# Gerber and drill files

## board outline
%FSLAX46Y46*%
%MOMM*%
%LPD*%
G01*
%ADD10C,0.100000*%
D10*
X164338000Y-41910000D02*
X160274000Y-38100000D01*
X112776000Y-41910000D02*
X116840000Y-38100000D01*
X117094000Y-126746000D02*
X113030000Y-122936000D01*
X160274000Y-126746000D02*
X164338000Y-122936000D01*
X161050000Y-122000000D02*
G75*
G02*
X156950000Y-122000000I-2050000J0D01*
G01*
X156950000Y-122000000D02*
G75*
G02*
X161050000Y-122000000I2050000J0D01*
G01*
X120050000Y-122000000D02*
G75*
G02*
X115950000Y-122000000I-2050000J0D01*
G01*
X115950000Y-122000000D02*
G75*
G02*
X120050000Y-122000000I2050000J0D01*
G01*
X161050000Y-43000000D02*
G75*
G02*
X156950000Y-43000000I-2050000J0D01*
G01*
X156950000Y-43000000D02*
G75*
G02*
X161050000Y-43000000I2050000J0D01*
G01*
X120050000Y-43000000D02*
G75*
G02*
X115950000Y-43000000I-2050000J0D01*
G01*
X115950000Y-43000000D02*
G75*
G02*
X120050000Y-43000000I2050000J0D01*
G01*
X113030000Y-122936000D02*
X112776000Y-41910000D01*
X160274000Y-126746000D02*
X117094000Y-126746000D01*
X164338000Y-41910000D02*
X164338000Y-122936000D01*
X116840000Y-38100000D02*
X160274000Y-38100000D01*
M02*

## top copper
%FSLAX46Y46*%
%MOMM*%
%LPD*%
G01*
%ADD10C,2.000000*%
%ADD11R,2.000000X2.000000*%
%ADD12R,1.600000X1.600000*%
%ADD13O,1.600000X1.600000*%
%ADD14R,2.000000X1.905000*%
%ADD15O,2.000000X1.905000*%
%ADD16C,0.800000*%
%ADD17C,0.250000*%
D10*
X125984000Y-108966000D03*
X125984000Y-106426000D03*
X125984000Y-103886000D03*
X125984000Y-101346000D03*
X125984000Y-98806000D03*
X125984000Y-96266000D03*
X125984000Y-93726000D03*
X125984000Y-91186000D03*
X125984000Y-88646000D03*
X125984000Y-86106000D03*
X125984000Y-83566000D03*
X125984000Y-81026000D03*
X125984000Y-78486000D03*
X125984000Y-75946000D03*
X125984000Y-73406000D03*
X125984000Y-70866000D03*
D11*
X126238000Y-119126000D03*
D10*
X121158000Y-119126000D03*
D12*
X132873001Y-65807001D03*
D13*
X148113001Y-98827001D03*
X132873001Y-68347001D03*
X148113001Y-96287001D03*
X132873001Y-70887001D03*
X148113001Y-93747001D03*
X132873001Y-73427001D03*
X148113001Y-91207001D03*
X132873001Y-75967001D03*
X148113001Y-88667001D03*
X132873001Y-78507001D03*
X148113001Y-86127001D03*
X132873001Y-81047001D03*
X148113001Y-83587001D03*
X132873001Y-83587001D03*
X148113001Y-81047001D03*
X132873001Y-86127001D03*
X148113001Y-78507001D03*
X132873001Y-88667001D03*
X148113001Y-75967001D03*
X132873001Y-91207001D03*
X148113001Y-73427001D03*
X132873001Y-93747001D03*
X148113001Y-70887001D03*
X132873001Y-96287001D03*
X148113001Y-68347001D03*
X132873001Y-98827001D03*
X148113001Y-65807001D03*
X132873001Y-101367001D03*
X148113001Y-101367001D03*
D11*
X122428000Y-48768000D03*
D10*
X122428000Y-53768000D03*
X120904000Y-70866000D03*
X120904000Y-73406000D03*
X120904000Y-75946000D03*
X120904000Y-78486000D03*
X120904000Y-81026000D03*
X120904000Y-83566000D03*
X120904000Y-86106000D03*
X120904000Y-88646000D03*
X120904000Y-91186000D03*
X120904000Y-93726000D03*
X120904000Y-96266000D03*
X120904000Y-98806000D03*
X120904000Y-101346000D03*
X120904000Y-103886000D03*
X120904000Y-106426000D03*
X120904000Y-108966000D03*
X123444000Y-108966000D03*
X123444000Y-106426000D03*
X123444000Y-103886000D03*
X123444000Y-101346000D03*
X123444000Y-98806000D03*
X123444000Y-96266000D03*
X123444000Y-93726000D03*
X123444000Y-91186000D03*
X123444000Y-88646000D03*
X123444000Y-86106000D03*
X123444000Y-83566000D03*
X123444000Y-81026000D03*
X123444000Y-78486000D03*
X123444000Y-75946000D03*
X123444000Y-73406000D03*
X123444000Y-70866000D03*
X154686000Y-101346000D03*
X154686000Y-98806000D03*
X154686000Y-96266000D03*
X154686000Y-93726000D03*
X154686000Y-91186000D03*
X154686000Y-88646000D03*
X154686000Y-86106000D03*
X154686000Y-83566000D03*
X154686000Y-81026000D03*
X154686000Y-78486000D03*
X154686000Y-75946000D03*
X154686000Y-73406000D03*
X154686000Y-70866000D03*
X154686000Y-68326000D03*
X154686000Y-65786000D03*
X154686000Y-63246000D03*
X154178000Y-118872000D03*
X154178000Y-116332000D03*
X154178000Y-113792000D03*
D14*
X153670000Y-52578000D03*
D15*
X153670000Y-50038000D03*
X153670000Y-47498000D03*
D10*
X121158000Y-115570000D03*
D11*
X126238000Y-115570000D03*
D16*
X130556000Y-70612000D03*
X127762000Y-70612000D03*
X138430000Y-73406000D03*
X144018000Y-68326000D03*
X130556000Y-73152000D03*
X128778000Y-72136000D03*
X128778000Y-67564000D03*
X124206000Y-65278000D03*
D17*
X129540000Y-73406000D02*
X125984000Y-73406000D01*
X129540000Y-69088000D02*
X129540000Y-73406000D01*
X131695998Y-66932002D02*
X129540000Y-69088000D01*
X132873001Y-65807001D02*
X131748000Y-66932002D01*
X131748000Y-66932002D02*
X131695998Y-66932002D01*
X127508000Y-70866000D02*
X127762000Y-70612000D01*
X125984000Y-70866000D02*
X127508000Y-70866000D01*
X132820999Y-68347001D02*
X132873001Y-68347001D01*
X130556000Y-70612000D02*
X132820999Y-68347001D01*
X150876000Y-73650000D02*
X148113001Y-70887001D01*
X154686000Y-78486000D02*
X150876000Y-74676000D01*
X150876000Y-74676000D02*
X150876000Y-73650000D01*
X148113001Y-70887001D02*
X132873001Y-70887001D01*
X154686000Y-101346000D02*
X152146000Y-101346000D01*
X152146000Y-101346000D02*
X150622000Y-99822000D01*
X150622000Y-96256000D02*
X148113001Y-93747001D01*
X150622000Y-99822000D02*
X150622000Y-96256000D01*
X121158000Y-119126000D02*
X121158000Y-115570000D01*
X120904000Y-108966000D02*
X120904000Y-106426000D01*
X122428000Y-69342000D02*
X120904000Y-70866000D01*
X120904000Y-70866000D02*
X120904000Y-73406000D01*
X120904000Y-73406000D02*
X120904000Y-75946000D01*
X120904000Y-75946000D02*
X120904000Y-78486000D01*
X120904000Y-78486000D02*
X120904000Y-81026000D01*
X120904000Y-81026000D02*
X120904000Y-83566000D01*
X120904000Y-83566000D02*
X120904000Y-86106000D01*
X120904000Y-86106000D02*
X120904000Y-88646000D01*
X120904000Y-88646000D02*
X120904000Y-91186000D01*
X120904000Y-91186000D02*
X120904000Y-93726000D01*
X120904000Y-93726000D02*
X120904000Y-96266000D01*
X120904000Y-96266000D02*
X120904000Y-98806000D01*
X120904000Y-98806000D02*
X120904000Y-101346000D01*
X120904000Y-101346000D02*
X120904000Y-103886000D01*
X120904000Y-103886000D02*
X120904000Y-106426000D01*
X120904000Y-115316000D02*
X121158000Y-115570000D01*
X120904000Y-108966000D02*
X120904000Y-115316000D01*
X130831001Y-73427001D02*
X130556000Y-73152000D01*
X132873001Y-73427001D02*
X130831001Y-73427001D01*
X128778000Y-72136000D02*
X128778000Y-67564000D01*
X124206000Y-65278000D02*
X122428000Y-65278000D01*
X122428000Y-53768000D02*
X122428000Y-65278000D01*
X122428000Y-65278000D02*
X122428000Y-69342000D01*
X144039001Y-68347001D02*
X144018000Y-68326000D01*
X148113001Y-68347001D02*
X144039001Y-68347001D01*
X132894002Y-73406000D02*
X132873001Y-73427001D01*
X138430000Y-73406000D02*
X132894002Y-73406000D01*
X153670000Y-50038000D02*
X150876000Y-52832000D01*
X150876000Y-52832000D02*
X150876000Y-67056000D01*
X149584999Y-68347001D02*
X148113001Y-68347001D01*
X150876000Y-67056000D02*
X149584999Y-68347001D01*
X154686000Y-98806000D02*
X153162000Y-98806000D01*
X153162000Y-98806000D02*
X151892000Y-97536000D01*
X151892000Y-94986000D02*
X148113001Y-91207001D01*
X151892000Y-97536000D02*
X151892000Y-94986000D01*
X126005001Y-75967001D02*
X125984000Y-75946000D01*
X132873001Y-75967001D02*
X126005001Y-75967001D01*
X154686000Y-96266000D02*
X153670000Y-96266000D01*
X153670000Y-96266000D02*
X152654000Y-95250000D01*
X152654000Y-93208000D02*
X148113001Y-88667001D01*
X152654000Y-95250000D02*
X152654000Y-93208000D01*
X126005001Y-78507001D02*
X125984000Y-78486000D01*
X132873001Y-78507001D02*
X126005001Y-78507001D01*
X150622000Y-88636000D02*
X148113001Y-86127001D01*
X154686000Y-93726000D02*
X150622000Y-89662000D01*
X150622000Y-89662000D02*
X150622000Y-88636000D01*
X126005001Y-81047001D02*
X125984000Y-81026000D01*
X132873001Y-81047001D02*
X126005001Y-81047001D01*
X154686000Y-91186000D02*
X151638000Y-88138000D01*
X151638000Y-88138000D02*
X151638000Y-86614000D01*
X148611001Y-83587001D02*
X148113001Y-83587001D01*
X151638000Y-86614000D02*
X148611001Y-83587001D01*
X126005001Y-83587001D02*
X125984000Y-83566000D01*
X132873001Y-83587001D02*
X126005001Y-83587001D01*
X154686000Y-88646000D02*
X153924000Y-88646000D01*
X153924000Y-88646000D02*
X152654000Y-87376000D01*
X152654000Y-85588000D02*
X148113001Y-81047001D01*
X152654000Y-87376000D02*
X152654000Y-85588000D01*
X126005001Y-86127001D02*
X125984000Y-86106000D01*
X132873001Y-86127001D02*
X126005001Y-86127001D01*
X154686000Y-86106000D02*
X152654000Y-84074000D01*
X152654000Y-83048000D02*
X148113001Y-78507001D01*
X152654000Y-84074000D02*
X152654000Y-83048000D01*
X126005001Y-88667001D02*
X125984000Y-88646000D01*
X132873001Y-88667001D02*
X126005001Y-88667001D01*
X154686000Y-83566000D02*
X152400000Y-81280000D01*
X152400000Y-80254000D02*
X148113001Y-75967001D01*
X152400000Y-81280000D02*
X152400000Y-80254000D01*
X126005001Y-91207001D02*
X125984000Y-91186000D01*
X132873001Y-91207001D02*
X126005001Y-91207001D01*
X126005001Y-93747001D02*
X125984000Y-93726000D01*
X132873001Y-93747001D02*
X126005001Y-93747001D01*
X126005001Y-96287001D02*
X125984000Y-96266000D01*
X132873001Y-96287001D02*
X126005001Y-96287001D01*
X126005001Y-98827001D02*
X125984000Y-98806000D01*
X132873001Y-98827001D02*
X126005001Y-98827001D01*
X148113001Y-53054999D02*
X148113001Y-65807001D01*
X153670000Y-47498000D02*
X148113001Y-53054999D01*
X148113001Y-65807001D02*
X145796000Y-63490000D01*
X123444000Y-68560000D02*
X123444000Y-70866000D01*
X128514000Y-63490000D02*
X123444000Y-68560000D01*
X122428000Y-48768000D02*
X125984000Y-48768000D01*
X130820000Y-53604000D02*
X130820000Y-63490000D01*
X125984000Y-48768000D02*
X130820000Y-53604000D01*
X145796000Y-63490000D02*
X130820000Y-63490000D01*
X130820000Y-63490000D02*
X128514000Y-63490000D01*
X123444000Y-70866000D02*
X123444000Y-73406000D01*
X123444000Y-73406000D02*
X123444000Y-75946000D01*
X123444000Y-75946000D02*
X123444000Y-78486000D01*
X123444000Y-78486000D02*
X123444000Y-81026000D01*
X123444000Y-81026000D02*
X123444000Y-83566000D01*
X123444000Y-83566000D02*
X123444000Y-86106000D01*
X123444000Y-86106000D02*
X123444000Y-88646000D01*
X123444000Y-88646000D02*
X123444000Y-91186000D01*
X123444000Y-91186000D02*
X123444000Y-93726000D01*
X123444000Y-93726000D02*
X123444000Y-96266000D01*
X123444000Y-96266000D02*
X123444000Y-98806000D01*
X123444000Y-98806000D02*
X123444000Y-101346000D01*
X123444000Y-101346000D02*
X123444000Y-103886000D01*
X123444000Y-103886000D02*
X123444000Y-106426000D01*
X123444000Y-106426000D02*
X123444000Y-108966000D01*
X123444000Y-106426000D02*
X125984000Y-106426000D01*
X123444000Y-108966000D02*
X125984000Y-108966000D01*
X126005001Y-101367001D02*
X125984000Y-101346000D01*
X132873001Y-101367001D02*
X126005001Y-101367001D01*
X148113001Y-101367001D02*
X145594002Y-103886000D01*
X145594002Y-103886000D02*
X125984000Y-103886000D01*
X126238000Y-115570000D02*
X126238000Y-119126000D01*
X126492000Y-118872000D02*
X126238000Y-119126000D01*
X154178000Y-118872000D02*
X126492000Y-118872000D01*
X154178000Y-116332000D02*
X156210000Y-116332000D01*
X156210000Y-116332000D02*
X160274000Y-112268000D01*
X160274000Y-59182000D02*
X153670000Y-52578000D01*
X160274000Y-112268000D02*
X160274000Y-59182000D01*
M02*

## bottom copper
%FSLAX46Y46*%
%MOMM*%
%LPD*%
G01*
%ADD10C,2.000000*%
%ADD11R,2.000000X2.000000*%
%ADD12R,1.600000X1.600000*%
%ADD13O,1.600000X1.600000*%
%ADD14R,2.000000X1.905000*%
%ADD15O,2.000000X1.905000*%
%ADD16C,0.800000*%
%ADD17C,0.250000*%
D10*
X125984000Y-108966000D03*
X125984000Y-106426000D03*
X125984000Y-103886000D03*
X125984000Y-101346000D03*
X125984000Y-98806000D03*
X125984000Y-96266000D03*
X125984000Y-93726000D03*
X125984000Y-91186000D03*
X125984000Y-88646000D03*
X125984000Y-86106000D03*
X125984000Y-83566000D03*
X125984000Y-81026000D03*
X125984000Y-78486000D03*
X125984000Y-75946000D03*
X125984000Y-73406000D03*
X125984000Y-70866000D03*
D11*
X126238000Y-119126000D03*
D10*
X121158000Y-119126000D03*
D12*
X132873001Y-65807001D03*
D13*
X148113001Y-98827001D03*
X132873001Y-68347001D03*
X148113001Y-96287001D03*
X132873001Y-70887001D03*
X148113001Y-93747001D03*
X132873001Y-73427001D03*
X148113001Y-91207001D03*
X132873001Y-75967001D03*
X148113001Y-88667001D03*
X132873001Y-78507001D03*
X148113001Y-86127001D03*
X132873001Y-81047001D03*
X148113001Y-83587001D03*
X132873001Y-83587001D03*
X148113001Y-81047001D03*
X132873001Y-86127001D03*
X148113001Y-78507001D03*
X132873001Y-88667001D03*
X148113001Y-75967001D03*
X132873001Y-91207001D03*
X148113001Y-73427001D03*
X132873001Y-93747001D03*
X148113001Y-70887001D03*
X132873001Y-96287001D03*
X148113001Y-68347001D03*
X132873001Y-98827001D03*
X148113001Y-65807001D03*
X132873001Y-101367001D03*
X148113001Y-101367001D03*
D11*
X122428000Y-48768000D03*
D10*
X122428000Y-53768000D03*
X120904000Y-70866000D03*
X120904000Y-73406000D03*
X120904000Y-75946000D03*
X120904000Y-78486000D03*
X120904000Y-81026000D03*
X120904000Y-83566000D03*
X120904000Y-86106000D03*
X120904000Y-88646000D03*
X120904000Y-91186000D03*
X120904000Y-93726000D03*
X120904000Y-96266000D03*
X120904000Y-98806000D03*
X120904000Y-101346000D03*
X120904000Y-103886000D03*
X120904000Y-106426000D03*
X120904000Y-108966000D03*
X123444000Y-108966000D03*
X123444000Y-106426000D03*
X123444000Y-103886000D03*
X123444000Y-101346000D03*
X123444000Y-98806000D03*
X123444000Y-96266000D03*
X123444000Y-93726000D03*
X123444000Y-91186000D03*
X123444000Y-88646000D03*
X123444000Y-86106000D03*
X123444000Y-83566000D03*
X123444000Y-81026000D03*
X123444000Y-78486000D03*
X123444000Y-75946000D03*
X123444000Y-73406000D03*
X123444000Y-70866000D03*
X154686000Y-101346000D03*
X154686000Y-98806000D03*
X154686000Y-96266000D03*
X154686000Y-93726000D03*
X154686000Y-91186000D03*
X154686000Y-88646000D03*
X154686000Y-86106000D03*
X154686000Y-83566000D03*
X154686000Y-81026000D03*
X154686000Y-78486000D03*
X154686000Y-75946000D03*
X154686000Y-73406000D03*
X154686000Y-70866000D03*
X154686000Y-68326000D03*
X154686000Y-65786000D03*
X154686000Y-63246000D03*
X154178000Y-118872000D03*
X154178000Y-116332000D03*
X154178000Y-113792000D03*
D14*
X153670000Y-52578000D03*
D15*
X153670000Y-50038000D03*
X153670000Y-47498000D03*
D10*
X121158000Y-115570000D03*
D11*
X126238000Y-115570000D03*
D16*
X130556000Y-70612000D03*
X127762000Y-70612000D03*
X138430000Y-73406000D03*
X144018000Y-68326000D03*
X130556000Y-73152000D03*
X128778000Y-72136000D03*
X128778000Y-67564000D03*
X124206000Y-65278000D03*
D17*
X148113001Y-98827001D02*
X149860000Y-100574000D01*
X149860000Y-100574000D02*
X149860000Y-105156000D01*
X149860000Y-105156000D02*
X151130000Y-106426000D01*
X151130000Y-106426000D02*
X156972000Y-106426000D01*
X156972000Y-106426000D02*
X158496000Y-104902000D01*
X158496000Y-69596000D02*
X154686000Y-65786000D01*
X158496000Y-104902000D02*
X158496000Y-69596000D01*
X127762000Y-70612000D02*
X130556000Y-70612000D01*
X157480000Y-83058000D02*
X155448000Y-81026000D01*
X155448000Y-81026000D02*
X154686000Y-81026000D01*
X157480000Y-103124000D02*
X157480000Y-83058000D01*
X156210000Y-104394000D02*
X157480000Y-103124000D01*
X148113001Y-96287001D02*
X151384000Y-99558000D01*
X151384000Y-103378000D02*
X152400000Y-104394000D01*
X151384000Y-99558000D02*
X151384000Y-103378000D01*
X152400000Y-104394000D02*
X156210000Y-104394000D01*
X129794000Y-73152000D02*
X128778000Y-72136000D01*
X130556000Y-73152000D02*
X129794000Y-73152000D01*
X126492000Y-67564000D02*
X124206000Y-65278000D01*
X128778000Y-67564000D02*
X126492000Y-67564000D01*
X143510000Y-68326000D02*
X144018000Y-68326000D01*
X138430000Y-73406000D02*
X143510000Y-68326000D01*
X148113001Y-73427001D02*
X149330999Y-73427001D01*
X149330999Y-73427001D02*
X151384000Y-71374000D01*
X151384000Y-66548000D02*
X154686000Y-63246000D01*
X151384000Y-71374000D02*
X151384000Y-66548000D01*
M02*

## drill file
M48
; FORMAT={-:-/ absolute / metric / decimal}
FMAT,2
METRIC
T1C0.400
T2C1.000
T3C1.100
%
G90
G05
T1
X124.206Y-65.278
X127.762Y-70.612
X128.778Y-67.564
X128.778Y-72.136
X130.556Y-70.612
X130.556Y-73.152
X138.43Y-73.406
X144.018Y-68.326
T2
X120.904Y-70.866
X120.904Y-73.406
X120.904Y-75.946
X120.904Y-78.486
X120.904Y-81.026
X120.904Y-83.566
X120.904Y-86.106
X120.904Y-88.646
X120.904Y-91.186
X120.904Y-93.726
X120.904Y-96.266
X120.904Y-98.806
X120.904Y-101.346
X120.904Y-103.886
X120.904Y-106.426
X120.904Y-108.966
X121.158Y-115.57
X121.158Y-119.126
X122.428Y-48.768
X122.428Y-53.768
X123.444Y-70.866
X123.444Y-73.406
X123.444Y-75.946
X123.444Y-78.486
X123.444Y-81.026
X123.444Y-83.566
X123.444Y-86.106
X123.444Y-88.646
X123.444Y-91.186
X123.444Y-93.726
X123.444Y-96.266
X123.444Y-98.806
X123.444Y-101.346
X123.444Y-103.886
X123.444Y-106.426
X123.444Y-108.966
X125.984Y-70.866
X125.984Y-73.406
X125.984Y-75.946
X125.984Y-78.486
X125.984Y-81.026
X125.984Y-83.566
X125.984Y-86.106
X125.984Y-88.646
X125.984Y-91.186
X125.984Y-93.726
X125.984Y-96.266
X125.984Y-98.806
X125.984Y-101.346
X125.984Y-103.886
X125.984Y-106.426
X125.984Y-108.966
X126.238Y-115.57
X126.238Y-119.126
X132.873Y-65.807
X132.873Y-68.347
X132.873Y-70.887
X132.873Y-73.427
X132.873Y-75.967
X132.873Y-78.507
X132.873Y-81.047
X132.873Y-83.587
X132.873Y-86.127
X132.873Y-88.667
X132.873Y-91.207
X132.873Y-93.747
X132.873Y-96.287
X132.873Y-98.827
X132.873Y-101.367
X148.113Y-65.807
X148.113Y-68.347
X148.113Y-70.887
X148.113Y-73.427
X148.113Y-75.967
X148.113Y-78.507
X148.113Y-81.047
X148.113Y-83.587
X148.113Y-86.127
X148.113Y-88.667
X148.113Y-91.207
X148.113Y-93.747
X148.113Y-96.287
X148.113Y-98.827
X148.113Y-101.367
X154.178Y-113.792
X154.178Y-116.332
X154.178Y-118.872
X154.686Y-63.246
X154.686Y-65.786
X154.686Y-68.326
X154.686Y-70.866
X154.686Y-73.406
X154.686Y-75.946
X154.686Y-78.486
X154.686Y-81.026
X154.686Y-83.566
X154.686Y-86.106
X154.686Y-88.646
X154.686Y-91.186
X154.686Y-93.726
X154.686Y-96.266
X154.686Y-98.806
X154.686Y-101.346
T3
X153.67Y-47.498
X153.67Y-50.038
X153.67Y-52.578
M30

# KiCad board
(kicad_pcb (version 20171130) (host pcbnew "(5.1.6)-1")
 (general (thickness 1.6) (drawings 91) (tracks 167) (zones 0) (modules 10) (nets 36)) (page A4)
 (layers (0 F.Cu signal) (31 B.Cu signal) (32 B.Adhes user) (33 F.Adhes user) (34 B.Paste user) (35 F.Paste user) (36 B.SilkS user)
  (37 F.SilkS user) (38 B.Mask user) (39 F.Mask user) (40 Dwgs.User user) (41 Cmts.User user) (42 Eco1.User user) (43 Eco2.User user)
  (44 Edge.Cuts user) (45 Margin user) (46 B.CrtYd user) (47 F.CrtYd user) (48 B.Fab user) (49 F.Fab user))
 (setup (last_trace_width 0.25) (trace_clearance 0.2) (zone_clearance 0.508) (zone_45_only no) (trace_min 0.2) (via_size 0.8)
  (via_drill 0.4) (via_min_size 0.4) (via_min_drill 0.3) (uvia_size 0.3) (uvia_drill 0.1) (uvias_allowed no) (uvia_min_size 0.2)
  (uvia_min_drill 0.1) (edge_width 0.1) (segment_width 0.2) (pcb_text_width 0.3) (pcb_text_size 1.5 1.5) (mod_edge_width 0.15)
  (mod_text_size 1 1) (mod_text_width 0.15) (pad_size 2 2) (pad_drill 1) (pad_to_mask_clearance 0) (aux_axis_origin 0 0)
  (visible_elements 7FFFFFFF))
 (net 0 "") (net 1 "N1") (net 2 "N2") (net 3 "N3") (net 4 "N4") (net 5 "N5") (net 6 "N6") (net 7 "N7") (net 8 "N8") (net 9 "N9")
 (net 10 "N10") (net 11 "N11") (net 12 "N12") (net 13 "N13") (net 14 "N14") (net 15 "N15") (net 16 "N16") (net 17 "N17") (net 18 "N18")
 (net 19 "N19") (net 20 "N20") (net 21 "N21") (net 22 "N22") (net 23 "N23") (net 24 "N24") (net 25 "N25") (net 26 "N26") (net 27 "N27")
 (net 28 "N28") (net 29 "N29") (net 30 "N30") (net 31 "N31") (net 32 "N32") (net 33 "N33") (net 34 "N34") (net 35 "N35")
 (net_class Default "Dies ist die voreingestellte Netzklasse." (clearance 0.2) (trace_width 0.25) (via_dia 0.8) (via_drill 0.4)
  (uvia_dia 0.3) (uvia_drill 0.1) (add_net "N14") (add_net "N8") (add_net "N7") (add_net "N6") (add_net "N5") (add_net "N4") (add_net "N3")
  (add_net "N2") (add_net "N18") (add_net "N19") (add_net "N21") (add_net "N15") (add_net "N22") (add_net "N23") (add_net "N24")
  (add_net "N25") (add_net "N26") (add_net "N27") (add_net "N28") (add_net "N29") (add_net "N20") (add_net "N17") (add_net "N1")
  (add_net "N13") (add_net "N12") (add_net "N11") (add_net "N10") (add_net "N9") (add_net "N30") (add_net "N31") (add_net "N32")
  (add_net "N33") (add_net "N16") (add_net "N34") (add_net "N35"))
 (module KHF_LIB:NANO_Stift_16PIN (layer F.Cu) (at 125.984 70.866 270)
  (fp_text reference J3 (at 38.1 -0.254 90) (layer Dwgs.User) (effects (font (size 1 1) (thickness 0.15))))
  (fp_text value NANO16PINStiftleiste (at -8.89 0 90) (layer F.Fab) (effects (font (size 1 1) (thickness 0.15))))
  (pad 16 thru_hole circle (at 38.1 0 270) (size 2 2) (drill 1) (layers *.Cu *.Mask) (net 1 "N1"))
  (pad 15 thru_hole circle (at 35.56 0 270) (size 2 2) (drill 1) (layers *.Cu *.Mask) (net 1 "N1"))
  (pad 14 thru_hole circle (at 33.02 0 270) (size 2 2) (drill 1) (layers *.Cu *.Mask) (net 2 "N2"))
  (pad 13 thru_hole circle (at 30.48 0 270) (size 2 2) (drill 1) (layers *.Cu *.Mask) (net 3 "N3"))
  (pad 12 thru_hole circle (at 27.94 0 270) (size 2 2) (drill 1) (layers *.Cu *.Mask) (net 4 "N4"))
  (pad 11 thru_hole circle (at 25.4 0 270) (size 2 2) (drill 1) (layers *.Cu *.Mask) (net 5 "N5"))
  (pad 10 thru_hole circle (at 22.86 0 270) (size 2 2) (drill 1) (layers *.Cu *.Mask) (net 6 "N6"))
  (pad 9 thru_hole circle (at 20.32 0 270) (size 2 2) (drill 1) (layers *.Cu *.Mask) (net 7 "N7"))
  (pad 8 thru_hole circle (at 17.78 0 270) (size 2 2) (drill 1) (layers *.Cu *.Mask) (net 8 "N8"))
  (pad 7 thru_hole circle (at 15.24 0 270) (size 2 2) (drill 1) (layers *.Cu *.Mask) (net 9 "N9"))
  (pad 6 thru_hole circle (at 12.7 0 270) (size 2 2) (drill 1) (layers *.Cu *.Mask) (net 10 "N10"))
  (pad 5 thru_hole circle (at 10.16 0 270) (size 2 2) (drill 1) (layers *.Cu *.Mask) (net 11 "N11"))
  (pad 4 thru_hole circle (at 7.62 0 270) (size 2 2) (drill 1) (layers *.Cu *.Mask) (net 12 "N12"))
  (pad 3 thru_hole circle (at 5.08 0 270) (size 2 2) (drill 1) (layers *.Cu *.Mask) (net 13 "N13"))
  (pad 2 thru_hole circle (at 2.54 0 270) (size 2 2) (drill 1) (layers *.Cu *.Mask) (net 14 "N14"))
  (pad 1 thru_hole circle (at 0 0 270) (size 2 2) (drill 1) (layers *.Cu *.Mask) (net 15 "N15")))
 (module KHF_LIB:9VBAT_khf (layer F.Cu) (at 121.158 119.126)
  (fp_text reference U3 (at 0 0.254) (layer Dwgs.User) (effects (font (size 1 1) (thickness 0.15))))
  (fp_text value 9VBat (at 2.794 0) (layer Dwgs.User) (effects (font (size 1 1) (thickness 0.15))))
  (pad 2 thru_hole rect (at 5.08 0) (size 2 2) (drill 1) (layers *.Cu *.Mask) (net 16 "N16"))
  (pad 1 thru_hole circle (at 0 0) (size 2 2) (drill 1) (layers *.Cu *.Mask) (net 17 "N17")))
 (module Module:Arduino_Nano (layer F.Cu) (at 132.873001 65.807001)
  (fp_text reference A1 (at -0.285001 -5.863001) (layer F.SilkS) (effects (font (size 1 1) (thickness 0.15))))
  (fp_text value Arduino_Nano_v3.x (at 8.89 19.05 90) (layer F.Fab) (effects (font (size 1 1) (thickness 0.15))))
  (pad 1 thru_hole rect (at 0 0) (size 1.6 1.6) (drill 1) (layers *.Cu *.Mask) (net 14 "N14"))
  (pad 17 thru_hole oval (at 15.24 33.02) (size 1.6 1.6) (drill 1) (layers *.Cu *.Mask) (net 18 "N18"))
  (pad 2 thru_hole oval (at 0 2.54) (size 1.6 1.6) (drill 1) (layers *.Cu *.Mask) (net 15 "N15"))
  (pad 18 thru_hole oval (at 15.24 30.48) (size 1.6 1.6) (drill 1) (layers *.Cu *.Mask) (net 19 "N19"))
  (pad 3 thru_hole oval (at 0 5.08) (size 1.6 1.6) (drill 1) (layers *.Cu *.Mask) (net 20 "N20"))
  (pad 19 thru_hole oval (at 15.24 27.94) (size 1.6 1.6) (drill 1) (layers *.Cu *.Mask) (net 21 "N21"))
  (pad 4 thru_hole oval (at 0 7.62) (size 1.6 1.6) (drill 1) (layers *.Cu *.Mask) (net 17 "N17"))
  (pad 20 thru_hole oval (at 15.24 25.4) (size 1.6 1.6) (drill 1) (layers *.Cu *.Mask) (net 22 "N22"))
  (pad 5 thru_hole oval (at 0 10.16) (size 1.6 1.6) (drill 1) (layers *.Cu *.Mask) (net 13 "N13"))
  (pad 21 thru_hole oval (at 15.24 22.86) (size 1.6 1.6) (drill 1) (layers *.Cu *.Mask) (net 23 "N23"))
  (pad 6 thru_hole oval (at 0 12.7) (size 1.6 1.6) (drill 1) (layers *.Cu *.Mask) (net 12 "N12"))
  (pad 22 thru_hole oval (at 15.24 20.32) (size 1.6 1.6) (drill 1) (layers *.Cu *.Mask) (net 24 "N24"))
  (pad 7 thru_hole oval (at 0 15.24) (size 1.6 1.6) (drill 1) (layers *.Cu *.Mask) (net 11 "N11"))
  (pad 23 thru_hole oval (at 15.24 17.78) (size 1.6 1.6) (drill 1) (layers *.Cu *.Mask) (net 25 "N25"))
  (pad 8 thru_hole oval (at 0 17.78) (size 1.6 1.6) (drill 1) (layers *.Cu *.Mask) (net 10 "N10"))
  (pad 24 thru_hole oval (at 15.24 15.24) (size 1.6 1.6) (drill 1) (layers *.Cu *.Mask) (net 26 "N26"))
  (pad 9 thru_hole oval (at 0 20.32) (size 1.6 1.6) (drill 1) (layers *.Cu *.Mask) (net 9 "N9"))
  (pad 25 thru_hole oval (at 15.24 12.7) (size 1.6 1.6) (drill 1) (layers *.Cu *.Mask) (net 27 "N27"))
  (pad 10 thru_hole oval (at 0 22.86) (size 1.6 1.6) (drill 1) (layers *.Cu *.Mask) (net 8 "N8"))
  (pad 26 thru_hole oval (at 15.24 10.16) (size 1.6 1.6) (drill 1) (layers *.Cu *.Mask) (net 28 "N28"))
  (pad 11 thru_hole oval (at 0 25.4) (size 1.6 1.6) (drill 1) (layers *.Cu *.Mask) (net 7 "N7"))
  (pad 27 thru_hole oval (at 15.24 7.62) (size 1.6 1.6) (drill 1) (layers *.Cu *.Mask) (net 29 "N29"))
  (pad 12 thru_hole oval (at 0 27.94) (size 1.6 1.6) (drill 1) (layers *.Cu *.Mask) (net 6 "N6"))
  (pad 28 thru_hole oval (at 15.24 5.08) (size 1.6 1.6) (drill 1) (layers *.Cu *.Mask) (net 20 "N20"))
  (pad 13 thru_hole oval (at 0 30.48) (size 1.6 1.6) (drill 1) (layers *.Cu *.Mask) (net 5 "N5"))
  (pad 29 thru_hole oval (at 15.24 2.54) (size 1.6 1.6) (drill 1) (layers *.Cu *.Mask) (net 17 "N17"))
  (pad 14 thru_hole oval (at 0 33.02) (size 1.6 1.6) (drill 1) (layers *.Cu *.Mask) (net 4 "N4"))
  (pad 30 thru_hole oval (at 15.24 0) (size 1.6 1.6) (drill 1) (layers *.Cu *.Mask) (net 1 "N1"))
  (pad 15 thru_hole oval (at 0 35.56) (size 1.6 1.6) (drill 1) (layers *.Cu *.Mask) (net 3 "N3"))
  (pad 16 thru_hole oval (at 15.24 35.56) (size 1.6 1.6) (drill 1) (layers *.Cu *.Mask) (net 2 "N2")))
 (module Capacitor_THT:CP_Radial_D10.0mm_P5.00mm (layer F.Cu) (at 122.428 48.768 270)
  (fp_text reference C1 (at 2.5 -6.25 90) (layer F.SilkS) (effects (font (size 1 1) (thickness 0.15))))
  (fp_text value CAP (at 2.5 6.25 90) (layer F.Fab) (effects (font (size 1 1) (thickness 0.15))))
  (pad 1 thru_hole rect (at 0 0 270) (size 2 2) (drill 1) (layers *.Cu *.Mask) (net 1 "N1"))
  (pad 2 thru_hole circle (at 5 0 270) (size 2 2) (drill 1) (layers *.Cu *.Mask) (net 17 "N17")))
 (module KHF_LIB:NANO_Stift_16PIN (layer F.Cu) (at 120.904 70.866 270)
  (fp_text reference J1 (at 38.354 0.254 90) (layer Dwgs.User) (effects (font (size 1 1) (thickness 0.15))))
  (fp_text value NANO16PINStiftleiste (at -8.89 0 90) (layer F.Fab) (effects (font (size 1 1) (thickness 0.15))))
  (pad 1 thru_hole circle (at 0 0 270) (size 2 2) (drill 1) (layers *.Cu *.Mask) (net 17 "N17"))
  (pad 2 thru_hole circle (at 2.54 0 270) (size 2 2) (drill 1) (layers *.Cu *.Mask) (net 17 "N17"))
  (pad 3 thru_hole circle (at 5.08 0 270) (size 2 2) (drill 1) (layers *.Cu *.Mask) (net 17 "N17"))
  (pad 4 thru_hole circle (at 7.62 0 270) (size 2 2) (drill 1) (layers *.Cu *.Mask) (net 17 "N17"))
  (pad 5 thru_hole circle (at 10.16 0 270) (size 2 2) (drill 1) (layers *.Cu *.Mask) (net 17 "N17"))
  (pad 6 thru_hole circle (at 12.7 0 270) (size 2 2) (drill 1) (layers *.Cu *.Mask) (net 17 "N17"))
  (pad 7 thru_hole circle (at 15.24 0 270) (size 2 2) (drill 1) (layers *.Cu *.Mask) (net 17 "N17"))
  (pad 8 thru_hole circle (at 17.78 0 270) (size 2 2) (drill 1) (layers *.Cu *.Mask) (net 17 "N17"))
  (pad 9 thru_hole circle (at 20.32 0 270) (size 2 2) (drill 1) (layers *.Cu *.Mask) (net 17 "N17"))
  (pad 10 thru_hole circle (at 22.86 0 270) (size 2 2) (drill 1) (layers *.Cu *.Mask) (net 17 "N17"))
  (pad 11 thru_hole circle (at 25.4 0 270) (size 2 2) (drill 1) (layers *.Cu *.Mask) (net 17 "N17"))
  (pad 12 thru_hole circle (at 27.94 0 270) (size 2 2) (drill 1) (layers *.Cu *.Mask) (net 17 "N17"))
  (pad 13 thru_hole circle (at 30.48 0 270) (size 2 2) (drill 1) (layers *.Cu *.Mask) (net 17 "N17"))
  (pad 14 thru_hole circle (at 33.02 0 270) (size 2 2) (drill 1) (layers *.Cu *.Mask) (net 17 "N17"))
  (pad 15 thru_hole circle (at 35.56 0 270) (size 2 2) (drill 1) (layers *.Cu *.Mask) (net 17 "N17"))
  (pad 16 thru_hole circle (at 38.1 0 270) (size 2 2) (drill 1) (layers *.Cu *.Mask) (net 17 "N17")))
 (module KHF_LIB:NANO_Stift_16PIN (layer F.Cu) (at 123.444 70.866 270)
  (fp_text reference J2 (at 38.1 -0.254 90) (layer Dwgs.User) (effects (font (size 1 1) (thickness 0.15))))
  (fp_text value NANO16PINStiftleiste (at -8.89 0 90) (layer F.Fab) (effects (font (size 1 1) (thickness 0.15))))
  (pad 16 thru_hole circle (at 38.1 0 270) (size 2 2) (drill 1) (layers *.Cu *.Mask) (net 1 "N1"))
  (pad 15 thru_hole circle (at 35.56 0 270) (size 2 2) (drill 1) (layers *.Cu *.Mask) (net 1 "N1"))
  (pad 14 thru_hole circle (at 33.02 0 270) (size 2 2) (drill 1) (layers *.Cu *.Mask) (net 1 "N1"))
  (pad 13 thru_hole circle (at 30.48 0 270) (size 2 2) (drill 1) (layers *.Cu *.Mask) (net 1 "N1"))
  (pad 12 thru_hole circle (at 27.94 0 270) (size 2 2) (drill 1) (layers *.Cu *.Mask) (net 1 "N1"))
  (pad 11 thru_hole circle (at 25.4 0 270) (size 2 2) (drill 1) (layers *.Cu *.Mask) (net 1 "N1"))
  (pad 10 thru_hole circle (at 22.86 0 270) (size 2 2) (drill 1) (layers *.Cu *.Mask) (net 1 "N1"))
  (pad 9 thru_hole circle (at 20.32 0 270) (size 2 2) (drill 1) (layers *.Cu *.Mask) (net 1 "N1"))
  (pad 8 thru_hole circle (at 17.78 0 270) (size 2 2) (drill 1) (layers *.Cu *.Mask) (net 1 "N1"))
  (pad 7 thru_hole circle (at 15.24 0 270) (size 2 2) (drill 1) (layers *.Cu *.Mask) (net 1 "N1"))
  (pad 6 thru_hole circle (at 12.7 0 270) (size 2 2) (drill 1) (layers *.Cu *.Mask) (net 1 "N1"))
  (pad 5 thru_hole circle (at 10.16 0 270) (size 2 2) (drill 1) (layers *.Cu *.Mask) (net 1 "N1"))
  (pad 4 thru_hole circle (at 7.62 0 270) (size 2 2) (drill 1) (layers *.Cu *.Mask) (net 1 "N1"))
  (pad 3 thru_hole circle (at 5.08 0 270) (size 2 2) (drill 1) (layers *.Cu *.Mask) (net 1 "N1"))
  (pad 2 thru_hole circle (at 2.54 0 270) (size 2 2) (drill 1) (layers *.Cu *.Mask) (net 1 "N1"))
  (pad 1 thru_hole circle (at 0 0 270) (size 2 2) (drill 1) (layers *.Cu *.Mask) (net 1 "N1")))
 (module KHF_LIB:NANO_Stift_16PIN (layer F.Cu) (at 154.686 101.346 90)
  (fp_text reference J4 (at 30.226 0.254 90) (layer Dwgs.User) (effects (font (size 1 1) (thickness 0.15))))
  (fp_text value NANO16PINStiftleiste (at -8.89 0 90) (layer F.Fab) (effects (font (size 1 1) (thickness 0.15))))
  (pad 1 thru_hole circle (at 0 0 90) (size 2 2) (drill 1) (layers *.Cu *.Mask) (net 21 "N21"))
  (pad 2 thru_hole circle (at 2.54 0 90) (size 2 2) (drill 1) (layers *.Cu *.Mask) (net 22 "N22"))
  (pad 3 thru_hole circle (at 5.08 0 90) (size 2 2) (drill 1) (layers *.Cu *.Mask) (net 23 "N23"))
  (pad 4 thru_hole circle (at 7.62 0 90) (size 2 2) (drill 1) (layers *.Cu *.Mask) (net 24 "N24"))
  (pad 5 thru_hole circle (at 10.16 0 90) (size 2 2) (drill 1) (layers *.Cu *.Mask) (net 25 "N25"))
  (pad 6 thru_hole circle (at 12.7 0 90) (size 2 2) (drill 1) (layers *.Cu *.Mask) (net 26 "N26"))
  (pad 7 thru_hole circle (at 15.24 0 90) (size 2 2) (drill 1) (layers *.Cu *.Mask) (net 27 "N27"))
  (pad 8 thru_hole circle (at 17.78 0 90) (size 2 2) (drill 1) (layers *.Cu *.Mask) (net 28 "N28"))
  (pad 9 thru_hole circle (at 20.32 0 90) (size 2 2) (drill 1) (layers *.Cu *.Mask) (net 19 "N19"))
  (pad 10 thru_hole circle (at 22.86 0 90) (size 2 2) (drill 1) (layers *.Cu *.Mask) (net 20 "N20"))
  (pad 11 thru_hole circle (at 25.4 0 90) (size 2 2) (drill 1) (layers *.Cu *.Mask) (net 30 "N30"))
  (pad 12 thru_hole circle (at 27.94 0 90) (size 2 2) (drill 1) (layers *.Cu *.Mask) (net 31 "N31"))
  (pad 13 thru_hole circle (at 30.48 0 90) (size 2 2) (drill 1) (layers *.Cu *.Mask) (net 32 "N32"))
  (pad 14 thru_hole circle (at 33.02 0 90) (size 2 2) (drill 1) (layers *.Cu *.Mask) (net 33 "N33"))
  (pad 15 thru_hole circle (at 35.56 0 90) (size 2 2) (drill 1) (layers *.Cu *.Mask) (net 18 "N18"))
  (pad 16 thru_hole circle (at 38.1 0 90) (size 2 2) (drill 1) (layers *.Cu *.Mask) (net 29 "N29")))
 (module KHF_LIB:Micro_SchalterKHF (layer F.Cu) (at 154.178 118.872 90)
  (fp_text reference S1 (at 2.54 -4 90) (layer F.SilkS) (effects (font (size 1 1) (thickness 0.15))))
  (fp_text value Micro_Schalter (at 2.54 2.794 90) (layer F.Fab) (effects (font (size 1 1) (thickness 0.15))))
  (pad 1 thru_hole circle (at 0 0 90) (size 2 2) (drill 1) (layers *.Cu *.Mask) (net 16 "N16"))
  (pad 2 thru_hole circle (at 2.54 0 90) (size 2 2) (drill 1) (layers *.Cu *.Mask) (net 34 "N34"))
  (pad 3 thru_hole circle (at 5.08 0 90) (size 2 2) (drill 1) (layers *.Cu *.Mask) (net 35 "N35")))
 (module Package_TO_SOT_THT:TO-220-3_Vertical (layer F.Cu) (at 153.67 52.578 90)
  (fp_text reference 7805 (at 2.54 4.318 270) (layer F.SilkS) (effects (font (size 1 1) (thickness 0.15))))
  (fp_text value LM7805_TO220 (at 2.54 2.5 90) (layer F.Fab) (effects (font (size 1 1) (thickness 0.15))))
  (pad 1 thru_hole rect (at 0 0 90) (size 1.905 2) (drill 1.1) (layers *.Cu *.Mask) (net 34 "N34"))
  (pad 2 thru_hole oval (at 2.54 0 90) (size 1.905 2) (drill 1.1) (layers *.Cu *.Mask) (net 17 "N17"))
  (pad 3 thru_hole oval (at 5.08 0 90) (size 1.905 2) (drill 1.1) (layers *.Cu *.Mask) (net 1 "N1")))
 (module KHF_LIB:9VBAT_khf (layer F.Cu) (at 121.158 115.57)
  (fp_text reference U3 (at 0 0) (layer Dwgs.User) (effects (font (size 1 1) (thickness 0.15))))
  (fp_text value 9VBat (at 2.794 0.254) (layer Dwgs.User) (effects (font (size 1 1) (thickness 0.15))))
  (pad 1 thru_hole circle (at 0 0) (size 2 2) (drill 1) (layers *.Cu *.Mask) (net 17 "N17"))
  (pad 2 thru_hole rect (at 5.08 0) (size 2 2) (drill 1) (layers *.Cu *.Mask) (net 16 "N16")))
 (gr_line (start 164.338 41.91) (end 160.274 38.1) (layer Edge.Cuts) (width 0.1))
 (gr_line (start 112.776 41.91) (end 116.84 38.1) (layer Edge.Cuts) (width 0.1))
 (gr_line (start 117.094 126.746) (end 113.03 122.936) (layer Edge.Cuts) (width 0.1))
 (gr_line (start 160.274 126.746) (end 164.338 122.936) (layer Edge.Cuts) (width 0.1))
 (gr_circle (center 159 122) (end 161.05 122) (layer Edge.Cuts) (width 0.1))
 (gr_circle (center 118 122) (end 120.05 122) (layer Edge.Cuts) (width 0.1))
 (gr_circle (center 159 43) (end 161.05 43) (layer Edge.Cuts) (width 0.1))
 (gr_circle (center 118 43) (end 120.05 43) (layer Edge.Cuts) (width 0.1))
 (gr_line (start 113.03 122.936) (end 112.776 41.91) (layer Edge.Cuts) (width 0.1))
 (gr_line (start 160.274 126.746) (end 117.094 126.746) (layer Edge.Cuts) (width 0.1))
 (gr_line (start 164.338 41.91) (end 164.338 122.936) (layer Edge.Cuts) (width 0.1))
 (gr_line (start 116.84 38.1) (end 160.274 38.1) (layer Edge.Cuts) (width 0.1))
 (segment (start 129.54 73.406) (end 125.984 73.406) (width 0.25) (layer F.Cu) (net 14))
 (segment (start 129.54 69.088) (end 129.54 73.406) (width 0.25) (layer F.Cu) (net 14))
 (segment (start 131.695998 66.932002) (end 129.54 69.088) (width 0.25) (layer F.Cu) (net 14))
 (segment (start 132.873001 65.807001) (end 131.748 66.932002) (width 0.25) (layer F.Cu) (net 14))
 (segment (start 131.748 66.932002) (end 131.695998 66.932002) (width 0.25) (layer F.Cu) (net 14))
 (segment (start 148.113001 98.827001) (end 149.86 100.574) (width 0.25) (layer B.Cu) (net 18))
 (segment (start 149.86 100.574) (end 149.86 105.156) (width 0.25) (layer B.Cu) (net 18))
 (segment (start 149.86 105.156) (end 151.13 106.426) (width 0.25) (layer B.Cu) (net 18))
 (segment (start 151.13 106.426) (end 156.972 106.426) (width 0.25) (layer B.Cu) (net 18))
 (segment (start 156.972 106.426) (end 158.496 104.902) (width 0.25) (layer B.Cu) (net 18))
 (segment (start 158.496 69.596) (end 154.686 65.786) (width 0.25) (layer B.Cu) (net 18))
 (segment (start 158.496 104.902) (end 158.496 69.596) (width 0.25) (layer B.Cu) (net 18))
 (via (at 130.556 70.612) (size 0.8) (drill 0.4) (layers F.Cu B.Cu) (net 15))
 (via (at 127.762 70.612) (size 0.8) (drill 0.4) (layers F.Cu B.Cu) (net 15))
 (segment (start 127.508 70.866) (end 127.762 70.612) (width 0.25) (layer F.Cu) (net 15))
 (segment (start 125.984 70.866) (end 127.508 70.866) (width 0.25) (layer F.Cu) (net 15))
 (segment (start 132.820999 68.347001) (end 132.873001 68.347001) (width 0.25) (layer F.Cu) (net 15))
 (segment (start 130.556 70.612) (end 132.820999 68.347001) (width 0.25) (layer F.Cu) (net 15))
 (segment (start 127.762 70.612) (end 130.556 70.612) (width 0.25) (layer B.Cu) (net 15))
 (segment (start 157.48 83.058) (end 155.448 81.026) (width 0.25) (layer B.Cu) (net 19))
 (segment (start 155.448 81.026) (end 154.686 81.026) (width 0.25) (layer B.Cu) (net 19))
 (segment (start 157.48 103.124) (end 157.48 83.058) (width 0.25) (layer B.Cu) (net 19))
 (segment (start 156.21 104.394) (end 157.48 103.124) (width 0.25) (layer B.Cu) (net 19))
 (segment (start 148.113001 96.287001) (end 151.384 99.558) (width 0.25) (layer B.Cu) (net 19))
 (segment (start 151.384 103.378) (end 152.4 104.394) (width 0.25) (layer B.Cu) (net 19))
 (segment (start 151.384 99.558) (end 151.384 103.378) (width 0.25) (layer B.Cu) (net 19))
 (segment (start 152.4 104.394) (end 156.21 104.394) (width 0.25) (layer B.Cu) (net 19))
 (segment (start 150.876 73.65) (end 148.113001 70.887001) (width 0.25) (layer F.Cu) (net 20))
 (segment (start 154.686 78.486) (end 150.876 74.676) (width 0.25) (layer F.Cu) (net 20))
 (segment (start 150.876 74.676) (end 150.876 73.65) (width 0.25) (layer F.Cu) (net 20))
 (segment (start 148.113001 70.887001) (end 132.873001 70.887001) (width 0.25) (layer F.Cu) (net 20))
 (segment (start 154.686 101.346) (end 152.146 101.346) (width 0.25) (layer F.Cu) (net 21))
 (segment (start 152.146 101.346) (end 150.622 99.822) (width 0.25) (layer F.Cu) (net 21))
 (segment (start 150.622 96.256) (end 148.113001 93.747001) (width 0.25) (layer F.Cu) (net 21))
 (segment (start 150.622 99.822) (end 150.622 96.256) (width 0.25) (layer F.Cu) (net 21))
 (via (at 138.43 73.406) (size 0.8) (drill 0.4) (layers F.Cu B.Cu) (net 17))
 (via (at 144.018 68.326) (size 0.8) (drill 0.4) (layers F.Cu B.Cu) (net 17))
 (via (at 130.556 73.152) (size 0.8) (drill 0.4) (layers F.Cu B.Cu) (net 17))
 (via (at 128.778 72.136) (size 0.8) (drill 0.4) (layers F.Cu B.Cu) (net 17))
 (via (at 128.778 67.564) (size 0.8) (drill 0.4) (layers F.Cu B.Cu) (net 17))
 (via (at 124.206 65.278) (size 0.8) (drill 0.4) (layers F.Cu B.Cu) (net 17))
 (segment (start 121.158 119.126) (end 121.158 115.57) (width 0.25) (layer F.Cu) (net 17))
 (segment (start 120.904 108.966) (end 120.904 106.426) (width 0.25) (layer F.Cu) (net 17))
 (segment (start 122.428 69.342) (end 120.904 70.866) (width 0.25) (layer F.Cu) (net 17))
 (segment (start 120.904 70.866) (end 120.904 73.406) (width 0.25) (layer F.Cu) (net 17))
 (segment (start 120.904 73.406) (end 120.904 75.946) (width 0.25) (layer F.Cu) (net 17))
 (segment (start 120.904 75.946) (end 120.904 78.486) (width 0.25) (layer F.Cu) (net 17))
 (segment (start 120.904 78.486) (end 120.904 81.026) (width 0.25) (layer F.Cu) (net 17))
 (segment (start 120.904 81.026) (end 120.904 83.566) (width 0.25) (layer F.Cu) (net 17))
 (segment (start 120.904 83.566) (end 120.904 86.106) (width 0.25) (layer F.Cu) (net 17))
 (segment (start 120.904 86.106) (end 120.904 88.646) (width 0.25) (layer F.Cu) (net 17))
 (segment (start 120.904 88.646) (end 120.904 91.186) (width 0.25) (layer F.Cu) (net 17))
 (segment (start 120.904 91.186) (end 120.904 93.726) (width 0.25) (layer F.Cu) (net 17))
 (segment (start 120.904 93.726) (end 120.904 96.266) (width 0.25) (layer F.Cu) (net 17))
 (segment (start 120.904 96.266) (end 120.904 98.806) (width 0.25) (layer F.Cu) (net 17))
 (segment (start 120.904 98.806) (end 120.904 101.346) (width 0.25) (layer F.Cu) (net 17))
 (segment (start 120.904 101.346) (end 120.904 103.886) (width 0.25) (layer F.Cu) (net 17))
 (segment (start 120.904 103.886) (end 120.904 106.426) (width 0.25) (layer F.Cu) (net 17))
 (segment (start 120.904 115.316) (end 121.158 115.57) (width 0.25) (layer F.Cu) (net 17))
 (segment (start 120.904 108.966) (end 120.904 115.316) (width 0.25) (layer F.Cu) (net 17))
 (segment (start 129.794 73.152) (end 128.778 72.136) (width 0.25) (layer B.Cu) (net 17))
 (segment (start 130.556 73.152) (end 129.794 73.152) (width 0.25) (layer B.Cu) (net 17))
 (segment (start 126.492 67.564) (end 124.206 65.278) (width 0.25) (layer B.Cu) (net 17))
 (segment (start 128.778 67.564) (end 126.492 67.564) (width 0.25) (layer B.Cu) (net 17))
 (segment (start 130.831001 73.427001) (end 130.556 73.152) (width 0.25) (layer F.Cu) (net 17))
 (segment (start 132.873001 73.427001) (end 130.831001 73.427001) (width 0.25) (layer F.Cu) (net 17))
 (segment (start 128.778 72.136) (end 128.778 67.564) (width 0.25) (layer F.Cu) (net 17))
 (segment (start 124.206 65.278) (end 122.428 65.278) (width 0.25) (layer F.Cu) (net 17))
 (segment (start 122.428 53.768) (end 122.428 65.278) (width 0.25) (layer F.Cu) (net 17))
 (segment (start 122.428 65.278) (end 122.428 69.342) (width 0.25) (layer F.Cu) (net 17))
 (segment (start 144.039001 68.347001) (end 144.018 68.326) (width 0.25) (layer F.Cu) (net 17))
 (segment (start 148.113001 68.347001) (end 144.039001 68.347001) (width 0.25) (layer F.Cu) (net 17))
 (segment (start 132.894002 73.406) (end 132.873001 73.427001) (width 0.25) (layer F.Cu) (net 17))
 (segment (start 138.43 73.406) (end 132.894002 73.406) (width 0.25) (layer F.Cu) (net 17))
 (segment (start 153.67 50.038) (end 150.876 52.832) (width 0.25) (layer F.Cu) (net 17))
 (segment (start 150.876 52.832) (end 150.876 67.056) (width 0.25) (layer F.Cu) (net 17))
 (segment (start 149.584999 68.347001) (end 148.113001 68.347001) (width 0.25) (layer F.Cu) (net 17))
 (segment (start 150.876 67.056) (end 149.584999 68.347001) (width 0.25) (layer F.Cu) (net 17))
 (segment (start 143.51 68.326) (end 144.018 68.326) (width 0.25) (layer B.Cu) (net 17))
 (segment (start 138.43 73.406) (end 143.51 68.326) (width 0.25) (layer B.Cu) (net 17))
 (segment (start 154.686 98.806) (end 153.162 98.806) (width 0.25) (layer F.Cu) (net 22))
 (segment (start 153.162 98.806) (end 151.892 97.536) (width 0.25) (layer F.Cu) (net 22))
 (segment (start 151.892 94.986) (end 148.113001 91.207001) (width 0.25) (layer F.Cu) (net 22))
 (segment (start 151.892 97.536) (end 151.892 94.986) (width 0.25) (layer F.Cu) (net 22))
 (segment (start 126.005001 75.967001) (end 125.984 75.946) (width 0.25) (layer F.Cu) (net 13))
 (segment (start 132.873001 75.967001) (end 126.005001 75.967001) (width 0.25) (layer F.Cu) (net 13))
 (segment (start 154.686 96.266) (end 153.67 96.266) (width 0.25) (layer F.Cu) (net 23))
 (segment (start 153.67 96.266) (end 152.654 95.25) (width 0.25) (layer F.Cu) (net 23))
 (segment (start 152.654 93.208) (end 148.113001 88.667001) (width 0.25) (layer F.Cu) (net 23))
 (segment (start 152.654 95.25) (end 152.654 93.208) (width 0.25) (layer F.Cu) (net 23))
 (segment (start 126.005001 78.507001) (end 125.984 78.486) (width 0.25) (layer F.Cu) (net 12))
 (segment (start 132.873001 78.507001) (end 126.005001 78.507001) (width 0.25) (layer F.Cu) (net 12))
 (segment (start 150.622 88.636) (end 148.113001 86.127001) (width 0.25) (layer F.Cu) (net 24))
 (segment (start 154.686 93.726) (end 150.622 89.662) (width 0.25) (layer F.Cu) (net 24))
 (segment (start 150.622 89.662) (end 150.622 88.636) (width 0.25) (layer F.Cu) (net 24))
 (segment (start 126.005001 81.047001) (end 125.984 81.026) (width 0.25) (layer F.Cu) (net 11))
 (segment (start 132.873001 81.047001) (end 126.005001 81.047001) (width 0.25) (layer F.Cu) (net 11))
 (segment (start 154.686 91.186) (end 151.638 88.138) (width 0.25) (layer F.Cu) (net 25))
 (segment (start 151.638 88.138) (end 151.638 86.614) (width 0.25) (layer F.Cu) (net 25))
 (segment (start 148.611001 83.587001) (end 148.113001 83.587001) (width 0.25) (layer F.Cu) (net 25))
 (segment (start 151.638 86.614) (end 148.611001 83.587001) (width 0.25) (layer F.Cu) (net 25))
 (segment (start 126.005001 83.587001) (end 125.984 83.566) (width 0.25) (layer F.Cu) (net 10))
 (segment (start 132.873001 83.587001) (end 126.005001 83.587001) (width 0.25) (layer F.Cu) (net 10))
 (segment (start 154.686 88.646) (end 153.924 88.646) (width 0.25) (layer F.Cu) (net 26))
 (segment (start 153.924 88.646) (end 152.654 87.376) (width 0.25) (layer F.Cu) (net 26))
 (segment (start 152.654 85.588) (end 148.113001 81.047001) (width 0.25) (layer F.Cu) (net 26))
 (segment (start 152.654 87.376) (end 152.654 85.588) (width 0.25) (layer F.Cu) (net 26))
 (segment (start 126.005001 86.127001) (end 125.984 86.106) (width 0.25) (layer F.Cu) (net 9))
 (segment (start 132.873001 86.127001) (end 126.005001 86.127001) (width 0.25) (layer F.Cu) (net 9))
 (segment (start 154.686 86.106) (end 152.654 84.074) (width 0.25) (layer F.Cu) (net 27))
 (segment (start 152.654 83.048) (end 148.113001 78.507001) (width 0.25) (layer F.Cu) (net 27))
 (segment (start 152.654 84.074) (end 152.654 83.048) (width 0.25) (layer F.Cu) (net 27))
 (segment (start 126.005001 88.667001) (end 125.984 88.646) (width 0.25) (layer F.Cu) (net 8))
 (segment (start 132.873001 88.667001) (end 126.005001 88.667001) (width 0.25) (layer F.Cu) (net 8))
 (segment (start 154.686 83.566) (end 152.4 81.28) (width 0.25) (layer F.Cu) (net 28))
 (segment (start 152.4 80.254) (end 148.113001 75.967001) (width 0.25) (layer F.Cu) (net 28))
 (segment (start 152.4 81.28) (end 152.4 80.254) (width 0.25) (layer F.Cu) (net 28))
 (segment (start 126.005001 91.207001) (end 125.984 91.186) (width 0.25) (layer F.Cu) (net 7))
 (segment (start 132.873001 91.207001) (end 126.005001 91.207001) (width 0.25) (layer F.Cu) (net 7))
 (segment (start 148.113001 73.427001) (end 149.330999 73.427001) (width 0.25) (layer B.Cu) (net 29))
 (segment (start 149.330999 73.427001) (end 151.384 71.374) (width 0.25) (layer B.Cu) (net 29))
 (segment (start 151.384 66.548) (end 154.686 63.246) (width 0.25) (layer B.Cu) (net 29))
 (segment (start 151.384 71.374) (end 151.384 66.548) (width 0.25) (layer B.Cu) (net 29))
 (segment (start 126.005001 93.747001) (end 125.984 93.726) (width 0.25) (layer F.Cu) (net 6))
 (segment (start 132.873001 93.747001) (end 126.005001 93.747001) (width 0.25) (layer F.Cu) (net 6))
 (segment (start 126.005001 96.287001) (end 125.984 96.266) (width 0.25) (layer F.Cu) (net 5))
 (segment (start 132.873001 96.287001) (end 126.005001 96.287001) (width 0.25) (layer F.Cu) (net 5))
 (segment (start 126.005001 98.827001) (end 125.984 98.806) (width 0.25) (layer F.Cu) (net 4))
 (segment (start 132.873001 98.827001) (end 126.005001 98.827001) (width 0.25) (layer F.Cu) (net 4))
 (segment (start 148.113001 53.054999) (end 148.113001 65.807001) (width 0.25) (layer F.Cu) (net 1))
 (segment (start 153.67 47.498) (end 148.113001 53.054999) (width 0.25) (layer F.Cu) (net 1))
 (segment (start 148.113001 65.807001) (end 145.796 63.49) (width 0.25) (layer F.Cu) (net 1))
 (segment (start 123.444 68.56) (end 123.444 70.866) (width 0.25) (layer F.Cu) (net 1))
 (segment (start 128.514 63.49) (end 123.444 68.56) (width 0.25) (layer F.Cu) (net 1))
 (segment (start 122.428 48.768) (end 125.984 48.768) (width 0.25) (layer F.Cu) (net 1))
 (segment (start 130.82 53.604) (end 130.82 63.49) (width 0.25) (layer F.Cu) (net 1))
 (segment (start 125.984 48.768) (end 130.82 53.604) (width 0.25) (layer F.Cu) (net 1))
 (segment (start 145.796 63.49) (end 130.82 63.49) (width 0.25) (layer F.Cu) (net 1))
 (segment (start 130.82 63.49) (end 128.514 63.49) (width 0.25) (layer F.Cu) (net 1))
 (segment (start 123.444 70.866) (end 123.444 73.406) (width 0.25) (layer F.Cu) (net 1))
 (segment (start 123.444 73.406) (end 123.444 75.946) (width 0.25) (layer F.Cu) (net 1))
 (segment (start 123.444 75.946) (end 123.444 78.486) (width 0.25) (layer F.Cu) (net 1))
 (segment (start 123.444 78.486) (end 123.444 81.026) (width 0.25) (layer F.Cu) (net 1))
 (segment (start 123.444 81.026) (end 123.444 83.566) (width 0.25) (layer F.Cu) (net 1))
 (segment (start 123.444 83.566) (end 123.444 86.106) (width 0.25) (layer F.Cu) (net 1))
 (segment (start 123.444 86.106) (end 123.444 88.646) (width 0.25) (layer F.Cu) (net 1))
 (segment (start 123.444 88.646) (end 123.444 91.186) (width 0.25) (layer F.Cu) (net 1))
 (segment (start 123.444 91.186) (end 123.444 93.726) (width 0.25) (layer F.Cu) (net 1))
 (segment (start 123.444 93.726) (end 123.444 96.266) (width 0.25) (layer F.Cu) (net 1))
 (segment (start 123.444 96.266) (end 123.444 98.806) (width 0.25) (layer F.Cu) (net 1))
 (segment (start 123.444 98.806) (end 123.444 101.346) (width 0.25) (layer F.Cu) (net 1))
 (segment (start 123.444 101.346) (end 123.444 103.886) (width 0.25) (layer F.Cu) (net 1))
 (segment (start 123.444 103.886) (end 123.444 106.426) (width 0.25) (layer F.Cu) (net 1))
 (segment (start 123.444 106.426) (end 123.444 108.966) (width 0.25) (layer F.Cu) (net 1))
 (segment (start 123.444 106.426) (end 125.984 106.426) (width 0.25) (layer F.Cu) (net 1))
 (segment (start 123.444 108.966) (end 125.984 108.966) (width 0.25) (layer F.Cu) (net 1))
 (segment (start 126.005001 101.367001) (end 125.984 101.346) (width 0.25) (layer F.Cu) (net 3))
 (segment (start 132.873001 101.367001) (end 126.005001 101.367001) (width 0.25) (layer F.Cu) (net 3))
 (segment (start 148.113001 101.367001) (end 145.594002 103.886) (width 0.25) (layer F.Cu) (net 2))
 (segment (start 145.594002 103.886) (end 125.984 103.886) (width 0.25) (layer F.Cu) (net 2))
 (segment (start 126.238 115.57) (end 126.238 119.126) (width 0.25) (layer F.Cu) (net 16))
 (segment (start 126.492 118.872) (end 126.238 119.126) (width 0.25) (layer F.Cu) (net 16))
 (segment (start 154.178 118.872) (end 126.492 118.872) (width 0.25) (layer F.Cu) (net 16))
 (segment (start 154.178 116.332) (end 156.21 116.332) (width 0.25) (layer F.Cu) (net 34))
 (segment (start 156.21 116.332) (end 160.274 112.268) (width 0.25) (layer F.Cu) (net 34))
 (segment (start 160.274 59.182) (end 153.67 52.578) (width 0.25) (layer F.Cu) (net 34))
 (segment (start 160.274 112.268) (end 160.274 59.182) (width 0.25) (layer F.Cu) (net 34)))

